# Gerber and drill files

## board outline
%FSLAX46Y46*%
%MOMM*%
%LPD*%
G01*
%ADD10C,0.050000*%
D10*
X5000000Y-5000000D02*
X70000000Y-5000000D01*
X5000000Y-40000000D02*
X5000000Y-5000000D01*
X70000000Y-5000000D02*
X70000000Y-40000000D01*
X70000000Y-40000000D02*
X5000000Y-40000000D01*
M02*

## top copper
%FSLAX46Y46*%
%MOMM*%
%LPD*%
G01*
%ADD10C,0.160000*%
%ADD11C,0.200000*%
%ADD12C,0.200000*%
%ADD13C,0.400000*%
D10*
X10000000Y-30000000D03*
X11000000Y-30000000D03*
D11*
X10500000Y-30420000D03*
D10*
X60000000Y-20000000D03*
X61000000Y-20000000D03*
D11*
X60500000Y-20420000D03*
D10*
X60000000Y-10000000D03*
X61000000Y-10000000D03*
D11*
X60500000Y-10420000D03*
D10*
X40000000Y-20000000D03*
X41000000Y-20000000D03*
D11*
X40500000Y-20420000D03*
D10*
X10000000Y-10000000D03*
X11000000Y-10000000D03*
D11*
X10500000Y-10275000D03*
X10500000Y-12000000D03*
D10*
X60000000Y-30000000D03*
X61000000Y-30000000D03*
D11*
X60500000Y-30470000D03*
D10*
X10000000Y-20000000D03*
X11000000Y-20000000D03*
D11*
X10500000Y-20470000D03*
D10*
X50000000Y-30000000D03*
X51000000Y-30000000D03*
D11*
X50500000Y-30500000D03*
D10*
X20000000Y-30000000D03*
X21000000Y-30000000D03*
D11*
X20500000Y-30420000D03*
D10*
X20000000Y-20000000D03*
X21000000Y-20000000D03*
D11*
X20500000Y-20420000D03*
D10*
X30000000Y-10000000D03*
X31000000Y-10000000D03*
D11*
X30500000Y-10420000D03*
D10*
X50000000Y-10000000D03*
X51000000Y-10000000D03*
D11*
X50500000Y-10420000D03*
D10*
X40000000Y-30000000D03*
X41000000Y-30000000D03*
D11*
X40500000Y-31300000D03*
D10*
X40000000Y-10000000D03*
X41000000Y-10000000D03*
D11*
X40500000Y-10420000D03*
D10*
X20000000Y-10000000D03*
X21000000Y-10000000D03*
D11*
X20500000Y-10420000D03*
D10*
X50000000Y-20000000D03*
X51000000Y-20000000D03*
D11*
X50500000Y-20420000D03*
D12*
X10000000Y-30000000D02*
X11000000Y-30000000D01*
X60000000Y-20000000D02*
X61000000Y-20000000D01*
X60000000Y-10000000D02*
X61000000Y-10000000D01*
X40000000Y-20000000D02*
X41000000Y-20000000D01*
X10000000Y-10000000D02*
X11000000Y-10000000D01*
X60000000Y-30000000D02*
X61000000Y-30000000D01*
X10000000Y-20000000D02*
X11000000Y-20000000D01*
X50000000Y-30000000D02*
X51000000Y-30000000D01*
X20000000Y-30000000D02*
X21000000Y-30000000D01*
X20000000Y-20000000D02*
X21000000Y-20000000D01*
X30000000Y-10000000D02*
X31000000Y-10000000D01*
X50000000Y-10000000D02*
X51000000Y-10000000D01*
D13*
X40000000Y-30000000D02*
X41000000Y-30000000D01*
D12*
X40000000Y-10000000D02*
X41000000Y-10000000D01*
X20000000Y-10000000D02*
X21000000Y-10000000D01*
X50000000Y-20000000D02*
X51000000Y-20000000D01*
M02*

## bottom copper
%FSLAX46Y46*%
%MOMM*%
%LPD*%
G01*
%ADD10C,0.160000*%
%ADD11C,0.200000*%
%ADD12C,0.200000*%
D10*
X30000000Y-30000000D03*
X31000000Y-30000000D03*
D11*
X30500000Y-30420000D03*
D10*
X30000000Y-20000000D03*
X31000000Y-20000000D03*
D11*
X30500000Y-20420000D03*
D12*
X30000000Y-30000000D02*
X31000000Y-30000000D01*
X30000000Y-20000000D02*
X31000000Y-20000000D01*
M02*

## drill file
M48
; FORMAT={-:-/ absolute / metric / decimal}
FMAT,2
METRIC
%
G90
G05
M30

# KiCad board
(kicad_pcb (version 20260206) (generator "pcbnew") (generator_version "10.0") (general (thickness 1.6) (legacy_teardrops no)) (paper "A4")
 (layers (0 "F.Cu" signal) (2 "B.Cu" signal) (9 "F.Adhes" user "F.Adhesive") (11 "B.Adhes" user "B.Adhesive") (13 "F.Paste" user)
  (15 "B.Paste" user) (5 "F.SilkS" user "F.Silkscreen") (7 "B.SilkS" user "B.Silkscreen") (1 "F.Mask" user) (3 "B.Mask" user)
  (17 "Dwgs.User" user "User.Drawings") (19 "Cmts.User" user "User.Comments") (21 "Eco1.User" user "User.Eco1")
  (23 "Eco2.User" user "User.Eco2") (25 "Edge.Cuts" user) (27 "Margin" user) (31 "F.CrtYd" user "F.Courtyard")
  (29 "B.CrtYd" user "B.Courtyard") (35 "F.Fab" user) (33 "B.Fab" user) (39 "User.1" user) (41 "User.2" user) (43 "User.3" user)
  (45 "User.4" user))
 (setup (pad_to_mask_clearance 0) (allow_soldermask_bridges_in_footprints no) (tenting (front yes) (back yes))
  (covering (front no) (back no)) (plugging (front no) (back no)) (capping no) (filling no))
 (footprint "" (layer "F.Cu") (at 10 30)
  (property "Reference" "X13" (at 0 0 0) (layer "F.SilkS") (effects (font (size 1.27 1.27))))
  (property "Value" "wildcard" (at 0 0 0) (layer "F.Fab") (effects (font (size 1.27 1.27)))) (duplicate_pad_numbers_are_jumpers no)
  (pad "1" smd circle (at 0 0) (size 0.16 0.16) (layers "F.Cu") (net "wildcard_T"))
  (pad "2" smd circle (at 1 0) (size 0.16 0.16) (layers "F.Cu") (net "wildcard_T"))
  (pad "3" smd circle (at 0.5 0.42) (size 0.2 0.2) (layers "F.Cu") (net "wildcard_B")))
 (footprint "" (layer "F.Cu") (at 60 20)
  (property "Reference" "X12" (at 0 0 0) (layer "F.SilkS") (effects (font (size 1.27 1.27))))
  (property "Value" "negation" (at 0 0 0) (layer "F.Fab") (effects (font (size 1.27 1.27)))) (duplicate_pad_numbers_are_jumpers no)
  (pad "1" smd circle (at 0 0) (size 0.16 0.16) (layers "F.Cu") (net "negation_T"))
  (pad "2" smd circle (at 1 0) (size 0.16 0.16) (layers "F.Cu") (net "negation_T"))
  (pad "3" smd circle (at 0.5 0.42) (size 0.2 0.2) (layers "F.Cu") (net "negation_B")))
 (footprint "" (layer "F.Cu") (at 60 10)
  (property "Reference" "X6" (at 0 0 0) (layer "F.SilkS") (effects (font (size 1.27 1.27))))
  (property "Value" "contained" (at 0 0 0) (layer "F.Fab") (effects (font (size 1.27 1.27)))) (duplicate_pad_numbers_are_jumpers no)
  (pad "1" smd circle (at 0 0) (size 0.16 0.16) (layers "F.Cu") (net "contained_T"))
  (pad "2" smd circle (at 1 0) (size 0.16 0.16) (layers "F.Cu") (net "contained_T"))
  (pad "3" smd circle (at 0.5 0.42) (size 0.2 0.2) (layers "F.Cu") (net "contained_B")))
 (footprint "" (layer "F.Cu") (at 40 20)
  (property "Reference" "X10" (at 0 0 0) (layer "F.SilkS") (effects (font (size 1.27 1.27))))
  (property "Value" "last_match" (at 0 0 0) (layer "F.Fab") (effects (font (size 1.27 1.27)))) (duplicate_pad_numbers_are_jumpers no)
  (pad "1" smd circle (at 0 0) (size 0.16 0.16) (layers "F.Cu") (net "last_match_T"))
  (pad "2" smd circle (at 1 0) (size 0.16 0.16) (layers "F.Cu") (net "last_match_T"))
  (pad "3" smd circle (at 0.5 0.42) (size 0.2 0.2) (layers "F.Cu") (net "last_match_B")))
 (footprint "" (layer "F.Cu") (at 10 10)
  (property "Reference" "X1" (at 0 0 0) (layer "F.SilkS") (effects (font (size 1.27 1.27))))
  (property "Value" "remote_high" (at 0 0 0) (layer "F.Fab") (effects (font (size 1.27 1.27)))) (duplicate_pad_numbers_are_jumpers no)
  (pad "1" smd circle (at 0 0) (size 0.16 0.16) (layers "F.Cu") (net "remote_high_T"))
  (pad "2" smd circle (at 1 0) (size 0.16 0.16) (layers "F.Cu") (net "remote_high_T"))
  (pad "3" smd circle (at 0.5 0.275) (size 0.2 0.2) (layers "F.Cu") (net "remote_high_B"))
  (pad "4" smd circle (at 0.5 2) (size 0.2 0.2) (layers "F.Cu") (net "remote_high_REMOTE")))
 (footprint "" (layer "F.Cu") (at 60 30)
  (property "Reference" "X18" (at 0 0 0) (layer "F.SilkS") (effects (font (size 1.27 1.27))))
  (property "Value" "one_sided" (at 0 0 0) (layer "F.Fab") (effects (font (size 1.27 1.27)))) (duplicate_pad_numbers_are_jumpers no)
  (pad "1" smd circle (at 0 0) (size 0.16 0.16) (layers "F.Cu") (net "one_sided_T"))
  (pad "2" smd circle (at 1 0) (size 0.16 0.16) (layers "F.Cu") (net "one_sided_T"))
  (pad "3" smd circle (at 0.5 0.47) (size 0.2 0.2) (layers "F.Cu") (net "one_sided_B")))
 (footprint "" (layer "F.Cu") (at 10 20)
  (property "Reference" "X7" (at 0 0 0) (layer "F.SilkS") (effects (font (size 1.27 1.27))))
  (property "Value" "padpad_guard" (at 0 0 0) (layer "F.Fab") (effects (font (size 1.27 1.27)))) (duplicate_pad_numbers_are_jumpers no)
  (pad "1" smd circle (at 0 0) (size 0.16 0.16) (layers "F.Cu") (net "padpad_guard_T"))
  (pad "2" smd circle (at 1 0) (size 0.16 0.16) (layers "F.Cu") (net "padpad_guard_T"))
  (pad "3" smd circle (at 0.5 0.47) (size 0.2 0.2) (layers "F.Cu") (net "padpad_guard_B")))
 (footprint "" (layer "F.Cu") (at 50 30)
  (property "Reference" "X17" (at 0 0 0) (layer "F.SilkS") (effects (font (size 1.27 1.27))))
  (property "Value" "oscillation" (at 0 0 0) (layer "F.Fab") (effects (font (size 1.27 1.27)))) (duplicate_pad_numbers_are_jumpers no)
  (pad "1" smd circle (at 0 0) (size 0.16 0.16) (layers "F.Cu") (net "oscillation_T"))
  (pad "2" smd circle (at 1 0) (size 0.16 0.16) (layers "F.Cu") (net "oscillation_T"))
  (pad "3" smd circle (at 0.5 0.5) (size 0.2 0.2) (layers "F.Cu") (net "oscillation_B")))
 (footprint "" (layer "F.Cu") (at 20 30)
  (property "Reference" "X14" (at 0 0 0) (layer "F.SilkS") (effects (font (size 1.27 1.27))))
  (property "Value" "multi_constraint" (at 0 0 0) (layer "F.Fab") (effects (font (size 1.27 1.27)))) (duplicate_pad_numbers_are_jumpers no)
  (pad "1" smd circle (at 0 0) (size 0.16 0.16) (layers "F.Cu") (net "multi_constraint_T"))
  (pad "2" smd circle (at 1 0) (size 0.16 0.16) (layers "F.Cu") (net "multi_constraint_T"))
  (pad "3" smd circle (at 0.5 0.42) (size 0.2 0.2) (layers "F.Cu") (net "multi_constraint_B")))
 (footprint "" (layer "F.Cu") (at 30 30)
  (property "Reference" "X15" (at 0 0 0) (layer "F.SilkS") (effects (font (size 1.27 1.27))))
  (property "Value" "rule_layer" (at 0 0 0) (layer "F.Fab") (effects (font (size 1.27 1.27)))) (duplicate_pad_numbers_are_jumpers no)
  (pad "1" smd circle (at 0 0) (size 0.16 0.16) (layers "B.Cu") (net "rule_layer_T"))
  (pad "2" smd circle (at 1 0) (size 0.16 0.16) (layers "B.Cu") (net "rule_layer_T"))
  (pad "3" smd circle (at 0.5 0.42) (size 0.2 0.2) (layers "B.Cu") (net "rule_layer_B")))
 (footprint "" (layer "F.Cu") (at 20 20)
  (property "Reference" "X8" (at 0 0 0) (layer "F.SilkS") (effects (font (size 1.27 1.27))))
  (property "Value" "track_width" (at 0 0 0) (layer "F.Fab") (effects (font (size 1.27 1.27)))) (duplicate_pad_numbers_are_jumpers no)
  (pad "1" smd circle (at 0 0) (size 0.16 0.16) (layers "F.Cu") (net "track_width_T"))
  (pad "2" smd circle (at 1 0) (size 0.16 0.16) (layers "F.Cu") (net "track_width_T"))
  (pad "3" smd circle (at 0.5 0.42) (size 0.2 0.2) (layers "F.Cu") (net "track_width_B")))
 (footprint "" (layer "F.Cu") (at 30 10)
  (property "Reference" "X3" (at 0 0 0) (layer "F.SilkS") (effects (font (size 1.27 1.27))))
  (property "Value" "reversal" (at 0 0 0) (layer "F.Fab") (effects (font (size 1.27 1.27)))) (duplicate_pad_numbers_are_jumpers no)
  (pad "1" smd circle (at 0 0) (size 0.16 0.16) (layers "F.Cu") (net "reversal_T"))
  (pad "2" smd circle (at 1 0) (size 0.16 0.16) (layers "F.Cu") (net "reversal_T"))
  (pad "3" smd circle (at 0.5 0.42) (size 0.2 0.2) (layers "F.Cu") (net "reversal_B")))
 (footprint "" (layer "F.Cu") (at 50 10)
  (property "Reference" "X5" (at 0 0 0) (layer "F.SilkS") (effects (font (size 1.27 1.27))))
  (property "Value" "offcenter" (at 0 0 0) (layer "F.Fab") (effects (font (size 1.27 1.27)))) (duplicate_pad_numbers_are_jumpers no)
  (pad "1" smd circle (at 0 0) (size 0.16 0.16) (layers "F.Cu") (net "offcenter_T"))
  (pad "2" smd circle (at 1 0) (size 0.16 0.16) (layers "F.Cu") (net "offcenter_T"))
  (pad "3" smd circle (at 0.5 0.42) (size 0.2 0.2) (layers "F.Cu") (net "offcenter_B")))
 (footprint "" (layer "F.Cu") (at 40 30)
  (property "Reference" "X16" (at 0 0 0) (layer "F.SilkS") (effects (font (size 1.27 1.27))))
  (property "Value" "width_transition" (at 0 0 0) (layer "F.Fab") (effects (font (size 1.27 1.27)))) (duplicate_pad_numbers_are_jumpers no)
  (pad "1" smd circle (at 0 0) (size 0.16 0.16) (layers "F.Cu") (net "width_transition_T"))
  (pad "2" smd circle (at 1 0) (size 0.16 0.16) (layers "F.Cu") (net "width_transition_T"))
  (pad "3" smd circle (at 0.5 1.3) (size 0.2 0.2) (layers "F.Cu") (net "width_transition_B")))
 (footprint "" (layer "F.Cu") (at 30 20)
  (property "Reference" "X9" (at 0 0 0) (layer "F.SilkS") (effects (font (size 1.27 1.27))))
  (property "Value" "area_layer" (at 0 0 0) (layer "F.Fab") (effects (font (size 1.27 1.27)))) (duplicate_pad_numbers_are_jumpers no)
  (pad "1" smd circle (at 0 0) (size 0.16 0.16) (layers "B.Cu") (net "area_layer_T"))
  (pad "2" smd circle (at 1 0) (size 0.16 0.16) (layers "B.Cu") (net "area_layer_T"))
  (pad "3" smd circle (at 0.5 0.42) (size 0.2 0.2) (layers "B.Cu") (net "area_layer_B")))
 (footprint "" (layer "F.Cu") (at 40 10)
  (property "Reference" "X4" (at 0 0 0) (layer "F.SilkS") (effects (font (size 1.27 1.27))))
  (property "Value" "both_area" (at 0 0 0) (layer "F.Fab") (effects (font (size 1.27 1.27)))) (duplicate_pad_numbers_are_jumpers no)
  (pad "1" smd circle (at 0 0) (size 0.16 0.16) (layers "F.Cu") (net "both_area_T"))
  (pad "2" smd circle (at 1 0) (size 0.16 0.16) (layers "F.Cu") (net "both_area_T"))
  (pad "3" smd circle (at 0.5 0.42) (size 0.2 0.2) (layers "F.Cu") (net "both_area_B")))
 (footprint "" (layer "F.Cu") (at 20 10)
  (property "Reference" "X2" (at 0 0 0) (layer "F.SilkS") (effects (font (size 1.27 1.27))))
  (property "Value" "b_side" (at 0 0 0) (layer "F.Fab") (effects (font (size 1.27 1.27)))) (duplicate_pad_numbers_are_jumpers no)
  (pad "1" smd circle (at 0 0) (size 0.16 0.16) (layers "F.Cu") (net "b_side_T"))
  (pad "2" smd circle (at 1 0) (size 0.16 0.16) (layers "F.Cu") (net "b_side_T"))
  (pad "3" smd circle (at 0.5 0.42) (size 0.2 0.2) (layers "F.Cu") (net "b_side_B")))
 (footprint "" (layer "F.Cu") (at 50 20)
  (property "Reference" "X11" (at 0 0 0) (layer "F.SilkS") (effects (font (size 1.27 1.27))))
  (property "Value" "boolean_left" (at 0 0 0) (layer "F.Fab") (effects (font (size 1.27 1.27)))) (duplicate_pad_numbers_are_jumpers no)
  (pad "1" smd circle (at 0 0) (size 0.16 0.16) (layers "F.Cu") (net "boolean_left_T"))
  (pad "2" smd circle (at 1 0) (size 0.16 0.16) (layers "F.Cu") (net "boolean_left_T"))
  (pad "3" smd circle (at 0.5 0.42) (size 0.2 0.2) (layers "F.Cu") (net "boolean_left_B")))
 (gr_line (start 5 5) (end 70 5) (stroke (width 0.05) (type default)) (layer "Edge.Cuts"))
 (gr_line (start 5 40) (end 5 5) (stroke (width 0.05) (type default)) (layer "Edge.Cuts"))
 (gr_line (start 70 5) (end 70 40) (stroke (width 0.05) (type default)) (layer "Edge.Cuts"))
 (gr_line (start 70 40) (end 5 40) (stroke (width 0.05) (type default)) (layer "Edge.Cuts"))
 (segment (start 10 30) (end 11 30) (width 0.2) (layer "F.Cu") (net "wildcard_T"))
 (segment (start 60 20) (end 61 20) (width 0.2) (layer "F.Cu") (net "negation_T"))
 (segment (start 60 10) (end 61 10) (width 0.2) (layer "F.Cu") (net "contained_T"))
 (segment (start 40 20) (end 41 20) (width 0.2) (layer "F.Cu") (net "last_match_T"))
 (segment (start 10 10) (end 11 10) (width 0.2) (layer "F.Cu") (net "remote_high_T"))
 (segment (start 60 30) (end 61 30) (width 0.2) (layer "F.Cu") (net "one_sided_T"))
 (segment (start 10 20) (end 11 20) (width 0.2) (layer "F.Cu") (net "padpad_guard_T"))
 (segment (start 50 30) (end 51 30) (width 0.2) (layer "F.Cu") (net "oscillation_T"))
 (segment (start 20 30) (end 21 30) (width 0.2) (layer "F.Cu") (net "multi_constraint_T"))
 (segment (start 30 30) (end 31 30) (width 0.2) (layer "B.Cu") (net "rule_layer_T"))
 (segment (start 20 20) (end 21 20) (width 0.2) (layer "F.Cu") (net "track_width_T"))
 (segment (start 30 10) (end 31 10) (width 0.2) (layer "F.Cu") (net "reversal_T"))
 (segment (start 50 10) (end 51 10) (width 0.2) (layer "F.Cu") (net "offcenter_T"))
 (segment (start 40 30) (end 41 30) (width 0.4) (layer "F.Cu") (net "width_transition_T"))
 (segment (start 30 20) (end 31 20) (width 0.2) (layer "B.Cu") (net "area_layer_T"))
 (segment (start 40 10) (end 41 10) (width 0.2) (layer "F.Cu") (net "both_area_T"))
 (segment (start 20 10) (end 21 10) (width 0.2) (layer "F.Cu") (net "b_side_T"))
 (segment (start 50 20) (end 51 20) (width 0.2) (layer "F.Cu") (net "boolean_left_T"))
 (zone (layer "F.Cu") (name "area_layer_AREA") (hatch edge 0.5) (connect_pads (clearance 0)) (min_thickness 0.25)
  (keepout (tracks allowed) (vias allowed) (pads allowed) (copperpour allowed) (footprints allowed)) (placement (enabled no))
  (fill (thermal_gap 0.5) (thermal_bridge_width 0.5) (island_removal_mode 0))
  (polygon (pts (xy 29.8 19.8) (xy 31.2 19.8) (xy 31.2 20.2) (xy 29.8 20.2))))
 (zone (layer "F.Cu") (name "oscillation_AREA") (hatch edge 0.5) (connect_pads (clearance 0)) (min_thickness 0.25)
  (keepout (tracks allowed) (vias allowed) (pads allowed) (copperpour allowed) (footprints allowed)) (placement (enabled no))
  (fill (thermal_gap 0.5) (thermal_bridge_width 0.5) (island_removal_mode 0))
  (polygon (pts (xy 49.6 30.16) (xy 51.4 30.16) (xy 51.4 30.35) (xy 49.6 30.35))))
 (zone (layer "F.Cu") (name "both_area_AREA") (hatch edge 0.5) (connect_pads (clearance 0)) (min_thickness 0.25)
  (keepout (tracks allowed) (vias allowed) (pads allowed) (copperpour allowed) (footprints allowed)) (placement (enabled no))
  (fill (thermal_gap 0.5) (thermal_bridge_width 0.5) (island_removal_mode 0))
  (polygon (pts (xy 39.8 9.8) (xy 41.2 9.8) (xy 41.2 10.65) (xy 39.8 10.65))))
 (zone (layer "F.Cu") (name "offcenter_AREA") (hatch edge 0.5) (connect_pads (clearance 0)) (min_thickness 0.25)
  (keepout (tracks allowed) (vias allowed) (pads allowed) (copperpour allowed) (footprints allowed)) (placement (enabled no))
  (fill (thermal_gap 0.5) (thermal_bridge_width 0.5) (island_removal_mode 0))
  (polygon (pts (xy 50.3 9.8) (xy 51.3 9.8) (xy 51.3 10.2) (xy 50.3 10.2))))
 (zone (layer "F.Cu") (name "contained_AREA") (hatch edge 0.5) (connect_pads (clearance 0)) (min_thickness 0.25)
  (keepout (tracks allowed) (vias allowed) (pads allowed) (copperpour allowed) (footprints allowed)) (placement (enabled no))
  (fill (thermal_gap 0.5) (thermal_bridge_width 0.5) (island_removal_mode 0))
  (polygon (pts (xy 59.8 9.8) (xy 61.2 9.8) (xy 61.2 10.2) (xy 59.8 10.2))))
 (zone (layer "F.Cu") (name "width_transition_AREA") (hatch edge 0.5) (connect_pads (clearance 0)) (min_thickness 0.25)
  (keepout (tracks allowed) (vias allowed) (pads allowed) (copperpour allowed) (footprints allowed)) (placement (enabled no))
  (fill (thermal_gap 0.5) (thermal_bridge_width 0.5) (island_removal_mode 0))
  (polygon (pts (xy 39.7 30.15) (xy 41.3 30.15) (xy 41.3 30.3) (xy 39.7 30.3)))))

